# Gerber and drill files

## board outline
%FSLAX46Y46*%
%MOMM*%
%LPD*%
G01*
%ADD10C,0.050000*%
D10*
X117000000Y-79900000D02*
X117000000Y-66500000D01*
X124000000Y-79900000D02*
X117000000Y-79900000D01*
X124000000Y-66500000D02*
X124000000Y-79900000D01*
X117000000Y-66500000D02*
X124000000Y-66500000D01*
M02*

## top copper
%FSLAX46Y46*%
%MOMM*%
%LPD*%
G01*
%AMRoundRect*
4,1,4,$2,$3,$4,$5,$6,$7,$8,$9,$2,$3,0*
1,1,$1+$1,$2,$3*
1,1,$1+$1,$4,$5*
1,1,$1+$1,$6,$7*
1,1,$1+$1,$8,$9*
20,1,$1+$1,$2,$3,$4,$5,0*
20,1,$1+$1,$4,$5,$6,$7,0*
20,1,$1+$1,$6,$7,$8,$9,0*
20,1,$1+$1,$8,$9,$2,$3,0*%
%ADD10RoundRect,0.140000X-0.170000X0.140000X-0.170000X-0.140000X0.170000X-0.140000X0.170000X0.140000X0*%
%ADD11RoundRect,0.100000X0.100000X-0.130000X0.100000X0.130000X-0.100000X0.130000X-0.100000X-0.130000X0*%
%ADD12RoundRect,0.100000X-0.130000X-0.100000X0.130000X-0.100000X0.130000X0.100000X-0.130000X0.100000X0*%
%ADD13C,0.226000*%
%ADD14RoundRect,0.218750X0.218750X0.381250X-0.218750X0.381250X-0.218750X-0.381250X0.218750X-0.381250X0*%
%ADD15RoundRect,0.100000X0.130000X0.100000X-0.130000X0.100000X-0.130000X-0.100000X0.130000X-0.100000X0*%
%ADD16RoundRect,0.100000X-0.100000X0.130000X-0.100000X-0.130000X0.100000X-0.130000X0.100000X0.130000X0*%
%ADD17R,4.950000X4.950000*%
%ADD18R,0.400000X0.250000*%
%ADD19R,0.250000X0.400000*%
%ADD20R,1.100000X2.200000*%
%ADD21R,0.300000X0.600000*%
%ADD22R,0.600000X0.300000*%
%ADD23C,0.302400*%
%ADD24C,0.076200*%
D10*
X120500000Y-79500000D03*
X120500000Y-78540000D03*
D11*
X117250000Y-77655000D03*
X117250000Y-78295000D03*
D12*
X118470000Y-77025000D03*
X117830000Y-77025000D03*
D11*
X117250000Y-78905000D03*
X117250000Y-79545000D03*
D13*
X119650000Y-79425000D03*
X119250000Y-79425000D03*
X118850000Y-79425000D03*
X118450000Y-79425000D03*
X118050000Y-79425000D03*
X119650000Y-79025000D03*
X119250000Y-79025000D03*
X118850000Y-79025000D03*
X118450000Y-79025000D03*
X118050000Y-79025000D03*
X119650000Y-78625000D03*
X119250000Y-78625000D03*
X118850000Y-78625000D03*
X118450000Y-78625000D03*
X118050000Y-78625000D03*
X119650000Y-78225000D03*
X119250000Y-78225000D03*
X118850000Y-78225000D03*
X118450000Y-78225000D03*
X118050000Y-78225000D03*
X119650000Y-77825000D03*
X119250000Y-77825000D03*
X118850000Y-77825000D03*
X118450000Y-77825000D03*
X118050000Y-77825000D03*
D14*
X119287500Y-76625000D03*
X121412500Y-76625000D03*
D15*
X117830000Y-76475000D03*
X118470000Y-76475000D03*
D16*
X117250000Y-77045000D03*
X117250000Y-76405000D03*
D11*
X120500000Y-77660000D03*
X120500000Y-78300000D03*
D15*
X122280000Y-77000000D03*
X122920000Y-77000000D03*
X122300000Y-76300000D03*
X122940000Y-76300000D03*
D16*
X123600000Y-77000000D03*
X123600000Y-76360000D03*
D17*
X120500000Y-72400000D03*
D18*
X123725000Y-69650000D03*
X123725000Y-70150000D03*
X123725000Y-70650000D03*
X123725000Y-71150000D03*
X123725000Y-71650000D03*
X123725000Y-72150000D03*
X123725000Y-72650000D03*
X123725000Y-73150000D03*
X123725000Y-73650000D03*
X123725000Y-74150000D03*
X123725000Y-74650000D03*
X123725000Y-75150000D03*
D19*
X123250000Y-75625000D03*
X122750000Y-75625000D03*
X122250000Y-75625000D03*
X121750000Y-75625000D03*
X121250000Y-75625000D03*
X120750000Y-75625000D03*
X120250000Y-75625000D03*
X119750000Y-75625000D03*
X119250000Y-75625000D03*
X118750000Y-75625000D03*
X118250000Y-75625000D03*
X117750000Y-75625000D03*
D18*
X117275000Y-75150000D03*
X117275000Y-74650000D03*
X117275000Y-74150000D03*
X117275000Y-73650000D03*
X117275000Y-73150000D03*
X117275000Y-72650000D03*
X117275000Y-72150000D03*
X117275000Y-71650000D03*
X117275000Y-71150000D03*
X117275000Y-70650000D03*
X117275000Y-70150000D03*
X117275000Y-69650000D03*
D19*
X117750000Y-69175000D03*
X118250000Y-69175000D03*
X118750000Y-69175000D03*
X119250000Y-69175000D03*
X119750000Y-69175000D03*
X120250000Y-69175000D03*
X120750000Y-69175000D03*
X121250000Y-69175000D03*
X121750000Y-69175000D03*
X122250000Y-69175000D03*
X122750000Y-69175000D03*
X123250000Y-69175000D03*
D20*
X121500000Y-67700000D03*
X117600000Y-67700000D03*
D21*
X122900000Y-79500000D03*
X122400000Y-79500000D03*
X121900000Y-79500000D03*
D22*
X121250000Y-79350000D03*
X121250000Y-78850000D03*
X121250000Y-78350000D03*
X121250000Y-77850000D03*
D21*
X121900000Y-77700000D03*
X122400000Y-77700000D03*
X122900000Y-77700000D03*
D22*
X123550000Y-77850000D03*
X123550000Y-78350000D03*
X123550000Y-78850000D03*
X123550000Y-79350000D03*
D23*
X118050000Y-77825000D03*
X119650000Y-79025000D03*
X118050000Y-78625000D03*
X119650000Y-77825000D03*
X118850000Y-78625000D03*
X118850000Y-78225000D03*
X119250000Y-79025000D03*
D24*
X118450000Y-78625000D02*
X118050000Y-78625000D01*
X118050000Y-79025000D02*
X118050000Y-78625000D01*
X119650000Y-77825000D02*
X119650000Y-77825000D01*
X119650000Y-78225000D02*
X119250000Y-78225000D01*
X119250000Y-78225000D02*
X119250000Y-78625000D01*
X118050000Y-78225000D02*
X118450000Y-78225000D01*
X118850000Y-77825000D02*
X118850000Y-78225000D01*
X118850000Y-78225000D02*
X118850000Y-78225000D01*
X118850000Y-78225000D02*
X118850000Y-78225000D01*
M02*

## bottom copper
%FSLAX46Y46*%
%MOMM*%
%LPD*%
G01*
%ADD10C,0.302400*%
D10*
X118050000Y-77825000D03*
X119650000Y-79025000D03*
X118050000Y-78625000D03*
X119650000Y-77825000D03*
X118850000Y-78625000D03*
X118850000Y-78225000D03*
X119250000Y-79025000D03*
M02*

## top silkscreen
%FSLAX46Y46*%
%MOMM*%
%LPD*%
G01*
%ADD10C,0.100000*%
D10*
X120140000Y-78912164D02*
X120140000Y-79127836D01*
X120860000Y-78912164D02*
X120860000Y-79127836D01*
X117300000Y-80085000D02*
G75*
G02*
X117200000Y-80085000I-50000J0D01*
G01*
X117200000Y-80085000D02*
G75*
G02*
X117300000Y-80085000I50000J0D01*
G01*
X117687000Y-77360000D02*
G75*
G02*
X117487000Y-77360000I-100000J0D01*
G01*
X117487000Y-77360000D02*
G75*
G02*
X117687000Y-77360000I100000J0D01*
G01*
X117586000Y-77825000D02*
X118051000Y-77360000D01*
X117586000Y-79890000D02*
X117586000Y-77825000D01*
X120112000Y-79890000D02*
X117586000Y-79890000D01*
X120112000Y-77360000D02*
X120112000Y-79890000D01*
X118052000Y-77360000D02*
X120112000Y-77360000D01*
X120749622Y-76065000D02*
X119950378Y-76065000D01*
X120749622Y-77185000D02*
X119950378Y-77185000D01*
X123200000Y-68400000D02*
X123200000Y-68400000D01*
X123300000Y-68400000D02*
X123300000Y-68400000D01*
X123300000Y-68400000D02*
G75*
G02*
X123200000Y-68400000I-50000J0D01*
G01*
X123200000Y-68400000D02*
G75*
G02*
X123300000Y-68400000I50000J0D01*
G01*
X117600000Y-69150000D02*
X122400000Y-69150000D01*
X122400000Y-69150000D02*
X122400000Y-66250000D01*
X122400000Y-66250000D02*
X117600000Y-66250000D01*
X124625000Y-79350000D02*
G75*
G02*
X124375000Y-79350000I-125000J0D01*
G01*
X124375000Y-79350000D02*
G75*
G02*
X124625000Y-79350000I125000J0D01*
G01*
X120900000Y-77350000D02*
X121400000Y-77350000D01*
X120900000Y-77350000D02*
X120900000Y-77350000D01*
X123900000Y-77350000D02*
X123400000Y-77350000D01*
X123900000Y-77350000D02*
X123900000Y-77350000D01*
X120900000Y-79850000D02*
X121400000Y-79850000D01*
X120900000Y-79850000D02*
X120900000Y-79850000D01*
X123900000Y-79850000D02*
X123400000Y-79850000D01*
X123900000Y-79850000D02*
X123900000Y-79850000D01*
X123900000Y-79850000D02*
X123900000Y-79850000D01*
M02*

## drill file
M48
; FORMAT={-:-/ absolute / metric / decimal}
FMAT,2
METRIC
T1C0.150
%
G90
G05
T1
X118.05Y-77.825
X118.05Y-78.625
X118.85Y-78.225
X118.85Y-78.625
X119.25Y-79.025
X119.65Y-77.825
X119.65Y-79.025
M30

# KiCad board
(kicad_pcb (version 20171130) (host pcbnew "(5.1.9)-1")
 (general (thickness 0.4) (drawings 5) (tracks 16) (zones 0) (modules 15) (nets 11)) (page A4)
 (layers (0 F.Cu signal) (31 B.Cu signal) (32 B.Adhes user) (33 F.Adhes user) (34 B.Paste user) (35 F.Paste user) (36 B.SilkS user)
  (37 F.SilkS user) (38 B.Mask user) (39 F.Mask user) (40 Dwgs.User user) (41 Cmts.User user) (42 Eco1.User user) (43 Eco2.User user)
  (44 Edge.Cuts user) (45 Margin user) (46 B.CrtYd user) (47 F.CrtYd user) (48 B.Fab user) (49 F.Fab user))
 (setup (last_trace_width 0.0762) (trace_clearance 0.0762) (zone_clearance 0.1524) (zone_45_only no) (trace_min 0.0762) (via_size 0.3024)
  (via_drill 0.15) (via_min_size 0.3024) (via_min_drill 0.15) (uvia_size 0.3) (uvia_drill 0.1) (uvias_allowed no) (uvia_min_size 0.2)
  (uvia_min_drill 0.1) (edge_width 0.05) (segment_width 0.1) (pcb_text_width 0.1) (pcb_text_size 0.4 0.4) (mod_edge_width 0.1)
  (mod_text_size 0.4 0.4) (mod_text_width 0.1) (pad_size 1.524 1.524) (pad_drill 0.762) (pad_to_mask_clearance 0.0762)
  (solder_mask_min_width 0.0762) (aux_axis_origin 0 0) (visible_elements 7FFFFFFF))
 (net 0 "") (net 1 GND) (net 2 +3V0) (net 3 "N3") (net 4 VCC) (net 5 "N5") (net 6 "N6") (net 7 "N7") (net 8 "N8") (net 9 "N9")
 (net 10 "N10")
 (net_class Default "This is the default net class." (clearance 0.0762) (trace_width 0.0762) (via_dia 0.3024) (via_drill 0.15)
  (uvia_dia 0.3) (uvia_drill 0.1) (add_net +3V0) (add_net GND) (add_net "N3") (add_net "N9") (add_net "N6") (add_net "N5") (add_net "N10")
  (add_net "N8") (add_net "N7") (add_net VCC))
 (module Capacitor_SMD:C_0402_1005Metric (layer F.Cu) (at 120.5 79.02 270)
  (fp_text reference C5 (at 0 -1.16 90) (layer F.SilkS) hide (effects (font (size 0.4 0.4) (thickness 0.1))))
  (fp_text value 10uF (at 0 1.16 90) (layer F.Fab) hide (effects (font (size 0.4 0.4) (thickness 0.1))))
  (fp_line (start -0.107836 0.36) (end 0.107836 0.36) (layer F.SilkS) (width 0.1))
  (fp_line (start -0.107836 -0.36) (end 0.107836 -0.36) (layer F.SilkS) (width 0.1))
  (pad 2 smd roundrect (at 0.48 0 270) (size 0.56 0.62) (layers F.Cu F.Paste F.Mask) (roundrect_rratio 0.25) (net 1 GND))
  (pad 1 smd roundrect (at -0.48 0 270) (size 0.56 0.62) (layers F.Cu F.Paste F.Mask) (roundrect_rratio 0.25) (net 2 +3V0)))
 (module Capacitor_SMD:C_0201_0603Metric (layer F.Cu) (at 117.25 77.975 90)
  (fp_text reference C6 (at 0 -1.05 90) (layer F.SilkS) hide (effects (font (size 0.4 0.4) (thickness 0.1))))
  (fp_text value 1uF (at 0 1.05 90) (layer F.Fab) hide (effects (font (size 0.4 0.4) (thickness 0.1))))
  (pad 2 smd roundrect (at 0.32 0 90) (size 0.46 0.4) (layers F.Cu F.Mask) (roundrect_rratio 0.25) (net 1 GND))
  (pad 1 smd roundrect (at -0.32 0 90) (size 0.46 0.4) (layers F.Cu F.Mask) (roundrect_rratio 0.25) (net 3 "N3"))
  (pad "" smd roundrect (at 0.345 0 90) (size 0.318 0.36) (layers F.Paste) (roundrect_rratio 0.25))
  (pad "" smd roundrect (at -0.345 0 90) (size 0.318 0.36) (layers F.Paste) (roundrect_rratio 0.25)))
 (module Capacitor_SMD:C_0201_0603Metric (layer F.Cu) (at 118.15 77.025)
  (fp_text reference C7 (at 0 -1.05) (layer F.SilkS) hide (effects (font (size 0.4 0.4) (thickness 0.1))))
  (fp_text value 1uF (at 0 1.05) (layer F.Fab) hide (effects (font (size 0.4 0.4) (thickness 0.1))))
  (pad 2 smd roundrect (at 0.32 0) (size 0.46 0.4) (layers F.Cu F.Mask) (roundrect_rratio 0.25) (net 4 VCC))
  (pad 1 smd roundrect (at -0.32 0) (size 0.46 0.4) (layers F.Cu F.Mask) (roundrect_rratio 0.25) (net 1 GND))
  (pad "" smd roundrect (at 0.345 0) (size 0.318 0.36) (layers F.Paste) (roundrect_rratio 0.25))
  (pad "" smd roundrect (at -0.345 0) (size 0.318 0.36) (layers F.Paste) (roundrect_rratio 0.25)))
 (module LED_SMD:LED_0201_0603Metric (layer F.Cu) (at 117.25 79.225 90)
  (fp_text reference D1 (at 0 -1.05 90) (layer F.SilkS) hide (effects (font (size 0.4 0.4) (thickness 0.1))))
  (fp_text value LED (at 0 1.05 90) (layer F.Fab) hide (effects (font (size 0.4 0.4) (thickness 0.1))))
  (fp_circle (center -0.86 0) (end -0.81 0) (layer F.SilkS) (width 0.1))
  (pad 2 smd roundrect (at 0.32 0 90) (size 0.46 0.4) (layers F.Cu F.Mask) (roundrect_rratio 0.25) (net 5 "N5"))
  (pad 1 smd roundrect (at -0.32 0 90) (size 0.46 0.4) (layers F.Cu F.Mask) (roundrect_rratio 0.25) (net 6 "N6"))
  (pad "" smd roundrect (at 0.345 0 90) (size 0.318 0.36) (layers F.Paste) (roundrect_rratio 0.25))
  (pad "" smd roundrect (at -0.345 0 90) (size 0.318 0.36) (layers F.Paste) (roundrect_rratio 0.25)))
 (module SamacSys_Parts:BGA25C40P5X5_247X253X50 (layer F.Cu) (at 118.85 78.625)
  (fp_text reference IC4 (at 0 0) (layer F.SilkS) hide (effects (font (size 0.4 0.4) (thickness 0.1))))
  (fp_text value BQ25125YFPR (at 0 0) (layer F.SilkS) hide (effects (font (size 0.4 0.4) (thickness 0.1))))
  (fp_circle (center -1.263 -1.265) (end -1.263 -1.165) (layer F.SilkS) (width 0.1))
  (fp_line (start -1.264 -0.8) (end -0.799 -1.265) (layer F.SilkS) (width 0.1))
  (fp_line (start -1.264 1.265) (end -1.264 -0.8) (layer F.SilkS) (width 0.1))
  (fp_line (start 1.262 1.265) (end -1.264 1.265) (layer F.SilkS) (width 0.1))
  (fp_line (start 1.262 -1.265) (end 1.262 1.265) (layer F.SilkS) (width 0.1))
  (fp_line (start -0.798 -1.265) (end 1.262 -1.265) (layer F.SilkS) (width 0.1))
  (pad E5 smd circle (at 0.8 0.8 90) (size 0.226 0.226) (layers F.Cu F.Paste F.Mask))
  (pad E4 smd circle (at 0.4 0.8 90) (size 0.226 0.226) (layers F.Cu F.Paste F.Mask))
  (pad E3 smd circle (at 0 0.8 90) (size 0.226 0.226) (layers F.Cu F.Paste F.Mask))
  (pad E2 smd circle (at -0.4 0.8 90) (size 0.226 0.226) (layers F.Cu F.Paste F.Mask))
  (pad E1 smd circle (at -0.8 0.8 90) (size 0.226 0.226) (layers F.Cu F.Paste F.Mask))
  (pad D5 smd circle (at 0.8 0.4 90) (size 0.226 0.226) (layers F.Cu F.Paste F.Mask) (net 1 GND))
  (pad D4 smd circle (at 0.4 0.4 90) (size 0.226 0.226) (layers F.Cu F.Paste F.Mask) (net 6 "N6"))
  (pad D3 smd circle (at 0 0.4 90) (size 0.226 0.226) (layers F.Cu F.Paste F.Mask))
  (pad D2 smd circle (at -0.4 0.4 90) (size 0.226 0.226) (layers F.Cu F.Paste F.Mask))
  (pad D1 smd circle (at -0.8 0.4 90) (size 0.226 0.226) (layers F.Cu F.Paste F.Mask) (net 1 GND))
  (pad C5 smd circle (at 0.8 0 90) (size 0.226 0.226) (layers F.Cu F.Paste F.Mask))
  (pad C4 smd circle (at 0.4 0 90) (size 0.226 0.226) (layers F.Cu F.Paste F.Mask) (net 2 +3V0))
  (pad C3 smd circle (at 0 0 90) (size 0.226 0.226) (layers F.Cu F.Paste F.Mask) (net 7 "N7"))
  (pad C2 smd circle (at -0.4 0 90) (size 0.226 0.226) (layers F.Cu F.Paste F.Mask) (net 1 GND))
  (pad C1 smd circle (at -0.8 0 90) (size 0.226 0.226) (layers F.Cu F.Paste F.Mask) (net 1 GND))
  (pad B5 smd circle (at 0.8 -0.4 90) (size 0.226 0.226) (layers F.Cu F.Paste F.Mask) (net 2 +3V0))
  (pad B4 smd circle (at 0.4 -0.4 90) (size 0.226 0.226) (layers F.Cu F.Paste F.Mask) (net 2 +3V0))
  (pad B3 smd circle (at 0 -0.4 90) (size 0.226 0.226) (layers F.Cu F.Paste F.Mask) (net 5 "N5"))
  (pad B2 smd circle (at -0.4 -0.4 90) (size 0.226 0.226) (layers F.Cu F.Paste F.Mask) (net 3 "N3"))
  (pad B1 smd circle (at -0.8 -0.4 90) (size 0.226 0.226) (layers F.Cu F.Paste F.Mask) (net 3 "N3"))
  (pad A5 smd circle (at 0.8 -0.8 90) (size 0.226 0.226) (layers F.Cu F.Paste F.Mask) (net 1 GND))
  (pad A4 smd circle (at 0.4 -0.8 90) (size 0.226 0.226) (layers F.Cu F.Paste F.Mask) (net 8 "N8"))
  (pad A3 smd circle (at 0 -0.8 90) (size 0.226 0.226) (layers F.Cu F.Paste F.Mask) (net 5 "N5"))
  (pad A2 smd circle (at -0.4 -0.8 90) (size 0.226 0.226) (layers F.Cu F.Paste F.Mask) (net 4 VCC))
  (pad A1 smd circle (at -0.8 -0.8 90) (size 0.226 0.226) (layers F.Cu F.Paste F.Mask) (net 1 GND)))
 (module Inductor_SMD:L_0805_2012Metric (layer F.Cu) (at 120.35 76.625 180)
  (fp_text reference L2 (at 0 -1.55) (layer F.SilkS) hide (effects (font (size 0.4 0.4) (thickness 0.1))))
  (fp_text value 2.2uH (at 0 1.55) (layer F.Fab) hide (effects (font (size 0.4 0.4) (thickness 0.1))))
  (fp_line (start -0.399622 0.56) (end 0.399622 0.56) (layer F.SilkS) (width 0.1))
  (fp_line (start -0.399622 -0.56) (end 0.399622 -0.56) (layer F.SilkS) (width 0.1))
  (pad 2 smd roundrect (at 1.0625 0 180) (size 0.875 1.2) (layers F.Cu F.Paste F.Mask) (roundrect_rratio 0.25) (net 8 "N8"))
  (pad 1 smd roundrect (at -1.0625 0 180) (size 0.875 1.2) (layers F.Cu F.Paste F.Mask) (roundrect_rratio 0.25) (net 2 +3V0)))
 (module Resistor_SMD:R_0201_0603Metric (layer F.Cu) (at 118.15 76.475 180)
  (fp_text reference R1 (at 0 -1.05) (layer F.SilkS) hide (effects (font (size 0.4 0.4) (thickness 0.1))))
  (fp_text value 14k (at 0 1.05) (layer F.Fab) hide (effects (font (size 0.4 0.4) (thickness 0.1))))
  (pad 2 smd roundrect (at 0.32 0 180) (size 0.46 0.4) (layers F.Cu F.Mask) (roundrect_rratio 0.25) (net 7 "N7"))
  (pad 1 smd roundrect (at -0.32 0 180) (size 0.46 0.4) (layers F.Cu F.Mask) (roundrect_rratio 0.25) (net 4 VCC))
  (pad "" smd roundrect (at 0.345 0 180) (size 0.318 0.36) (layers F.Paste) (roundrect_rratio 0.25))
  (pad "" smd roundrect (at -0.345 0 180) (size 0.318 0.36) (layers F.Paste) (roundrect_rratio 0.25)))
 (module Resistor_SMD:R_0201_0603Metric (layer F.Cu) (at 117.25 76.725 270)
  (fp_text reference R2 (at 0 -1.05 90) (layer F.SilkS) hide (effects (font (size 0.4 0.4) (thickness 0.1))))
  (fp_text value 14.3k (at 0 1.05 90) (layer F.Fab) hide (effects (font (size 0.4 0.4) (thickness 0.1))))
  (pad 2 smd roundrect (at 0.32 0 270) (size 0.46 0.4) (layers F.Cu F.Mask) (roundrect_rratio 0.25) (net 1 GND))
  (pad 1 smd roundrect (at -0.32 0 270) (size 0.46 0.4) (layers F.Cu F.Mask) (roundrect_rratio 0.25) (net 7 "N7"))
  (pad "" smd roundrect (at 0.345 0 270) (size 0.318 0.36) (layers F.Paste) (roundrect_rratio 0.25))
  (pad "" smd roundrect (at -0.345 0 270) (size 0.318 0.36) (layers F.Paste) (roundrect_rratio 0.25)))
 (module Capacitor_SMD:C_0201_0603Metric (layer F.Cu) (at 120.5 77.98 90)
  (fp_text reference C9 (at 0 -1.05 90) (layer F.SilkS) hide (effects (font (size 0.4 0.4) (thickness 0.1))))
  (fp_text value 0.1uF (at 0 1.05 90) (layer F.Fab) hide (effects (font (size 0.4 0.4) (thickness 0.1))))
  (pad 2 smd roundrect (at 0.32 0 90) (size 0.46 0.4) (layers F.Cu F.Mask) (roundrect_rratio 0.25) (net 1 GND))
  (pad 1 smd roundrect (at -0.32 0 90) (size 0.46 0.4) (layers F.Cu F.Mask) (roundrect_rratio 0.25) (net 2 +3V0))
  (pad "" smd roundrect (at 0.345 0 90) (size 0.318 0.36) (layers F.Paste) (roundrect_rratio 0.25))
  (pad "" smd roundrect (at -0.345 0 90) (size 0.318 0.36) (layers F.Paste) (roundrect_rratio 0.25)))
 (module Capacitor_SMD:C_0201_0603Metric (layer F.Cu) (at 122.6 77 180)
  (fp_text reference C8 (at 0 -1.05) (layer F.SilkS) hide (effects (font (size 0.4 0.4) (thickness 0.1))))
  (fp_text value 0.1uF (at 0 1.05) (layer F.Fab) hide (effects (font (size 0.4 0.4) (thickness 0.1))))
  (pad 2 smd roundrect (at 0.32 0 180) (size 0.46 0.4) (layers F.Cu F.Mask) (roundrect_rratio 0.25) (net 1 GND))
  (pad 1 smd roundrect (at -0.32 0 180) (size 0.46 0.4) (layers F.Cu F.Mask) (roundrect_rratio 0.25) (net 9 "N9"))
  (pad "" smd roundrect (at 0.345 0 180) (size 0.318 0.36) (layers F.Paste) (roundrect_rratio 0.25))
  (pad "" smd roundrect (at -0.345 0 180) (size 0.318 0.36) (layers F.Paste) (roundrect_rratio 0.25)))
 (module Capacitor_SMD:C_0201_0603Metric (layer F.Cu) (at 122.62 76.3 180)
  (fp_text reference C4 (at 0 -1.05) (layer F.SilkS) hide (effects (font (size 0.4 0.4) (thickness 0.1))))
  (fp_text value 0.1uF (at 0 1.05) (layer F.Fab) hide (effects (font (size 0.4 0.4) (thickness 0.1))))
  (pad 2 smd roundrect (at 0.32 0 180) (size 0.46 0.4) (layers F.Cu F.Mask) (roundrect_rratio 0.25) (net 1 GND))
  (pad 1 smd roundrect (at -0.32 0 180) (size 0.46 0.4) (layers F.Cu F.Mask) (roundrect_rratio 0.25) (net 2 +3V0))
  (pad "" smd roundrect (at 0.345 0 180) (size 0.318 0.36) (layers F.Paste) (roundrect_rratio 0.25))
  (pad "" smd roundrect (at -0.345 0 180) (size 0.318 0.36) (layers F.Paste) (roundrect_rratio 0.25)))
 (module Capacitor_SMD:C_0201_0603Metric (layer F.Cu) (at 123.6 76.68 270)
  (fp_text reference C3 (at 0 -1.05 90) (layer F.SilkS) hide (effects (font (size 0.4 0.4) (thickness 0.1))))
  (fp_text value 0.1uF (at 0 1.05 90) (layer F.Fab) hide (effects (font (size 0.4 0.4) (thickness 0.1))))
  (pad 2 smd roundrect (at 0.32 0 270) (size 0.46 0.4) (layers F.Cu F.Mask) (roundrect_rratio 0.25) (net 1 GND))
  (pad 1 smd roundrect (at -0.32 0 270) (size 0.46 0.4) (layers F.Cu F.Mask) (roundrect_rratio 0.25) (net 2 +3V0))
  (pad "" smd roundrect (at 0.345 0 270) (size 0.318 0.36) (layers F.Paste) (roundrect_rratio 0.25))
  (pad "" smd roundrect (at -0.345 0 270) (size 0.318 0.36) (layers F.Paste) (roundrect_rratio 0.25)))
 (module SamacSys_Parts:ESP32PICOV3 (layer F.Cu) (at 120.5 72.4 270)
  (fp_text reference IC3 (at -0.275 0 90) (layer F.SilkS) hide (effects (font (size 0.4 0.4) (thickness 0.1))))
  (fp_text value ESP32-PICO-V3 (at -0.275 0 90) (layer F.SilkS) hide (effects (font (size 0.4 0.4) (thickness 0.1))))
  (fp_line (start -4 -2.7) (end -4 -2.7) (layer F.SilkS) (width 0.1))
  (fp_line (start -4 -2.8) (end -4 -2.8) (layer F.SilkS) (width 0.1))
  (fp_arc (start -4 -2.75) (end -4 -2.7) (angle -180) (layer F.SilkS) (width 0.1))
  (fp_arc (start -4 -2.75) (end -4 -2.8) (angle -180) (layer F.SilkS) (width 0.1))
  (pad 49 smd rect (at 0 0 270) (size 4.95 4.95) (layers F.Cu F.Paste F.Mask) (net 1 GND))
  (pad 48 smd rect (at -2.75 -3.225 270) (size 0.25 0.4) (layers F.Cu F.Paste F.Mask))
  (pad 47 smd rect (at -2.25 -3.225 270) (size 0.25 0.4) (layers F.Cu F.Paste F.Mask))
  (pad 46 smd rect (at -1.75 -3.225 270) (size 0.25 0.4) (layers F.Cu F.Paste F.Mask) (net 2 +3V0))
  (pad 45 smd rect (at -1.25 -3.225 270) (size 0.25 0.4) (layers F.Cu F.Paste F.Mask))
  (pad 44 smd rect (at -0.75 -3.225 270) (size 0.25 0.4) (layers F.Cu F.Paste F.Mask))
  (pad 43 smd rect (at -0.25 -3.225 270) (size 0.25 0.4) (layers F.Cu F.Paste F.Mask) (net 2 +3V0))
  (pad 42 smd rect (at 0.25 -3.225 270) (size 0.25 0.4) (layers F.Cu F.Paste F.Mask))
  (pad 41 smd rect (at 0.75 -3.225 270) (size 0.25 0.4) (layers F.Cu F.Paste F.Mask))
  (pad 40 smd rect (at 1.25 -3.225 270) (size 0.25 0.4) (layers F.Cu F.Paste F.Mask))
  (pad 39 smd rect (at 1.75 -3.225 270) (size 0.25 0.4) (layers F.Cu F.Paste F.Mask))
  (pad 38 smd rect (at 2.25 -3.225 270) (size 0.25 0.4) (layers F.Cu F.Paste F.Mask))
  (pad 37 smd rect (at 2.75 -3.225 270) (size 0.25 0.4) (layers F.Cu F.Paste F.Mask) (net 2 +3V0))
  (pad 36 smd rect (at 3.225 -2.75) (size 0.25 0.4) (layers F.Cu F.Paste F.Mask))
  (pad 35 smd rect (at 3.225 -2.25) (size 0.25 0.4) (layers F.Cu F.Paste F.Mask))
  (pad 34 smd rect (at 3.225 -1.75) (size 0.25 0.4) (layers F.Cu F.Paste F.Mask))
  (pad 33 smd rect (at 3.225 -1.25) (size 0.25 0.4) (layers F.Cu F.Paste F.Mask))
  (pad 32 smd rect (at 3.225 -0.75) (size 0.25 0.4) (layers F.Cu F.Paste F.Mask))
  (pad 31 smd rect (at 3.225 -0.25) (size 0.25 0.4) (layers F.Cu F.Paste F.Mask))
  (pad 30 smd rect (at 3.225 0.25) (size 0.25 0.4) (layers F.Cu F.Paste F.Mask))
  (pad 29 smd rect (at 3.225 0.75) (size 0.25 0.4) (layers F.Cu F.Paste F.Mask))
  (pad 28 smd rect (at 3.225 1.25) (size 0.25 0.4) (layers F.Cu F.Paste F.Mask))
  (pad 27 smd rect (at 3.225 1.75) (size 0.25 0.4) (layers F.Cu F.Paste F.Mask))
  (pad 26 smd rect (at 3.225 2.25) (size 0.25 0.4) (layers F.Cu F.Paste F.Mask))
  (pad 25 smd rect (at 3.225 2.75) (size 0.25 0.4) (layers F.Cu F.Paste F.Mask))
  (pad 24 smd rect (at 2.75 3.225 270) (size 0.25 0.4) (layers F.Cu F.Paste F.Mask))
  (pad 23 smd rect (at 2.25 3.225 270) (size 0.25 0.4) (layers F.Cu F.Paste F.Mask))
  (pad 22 smd rect (at 1.75 3.225 270) (size 0.25 0.4) (layers F.Cu F.Paste F.Mask))
  (pad 21 smd rect (at 1.25 3.225 270) (size 0.25 0.4) (layers F.Cu F.Paste F.Mask))
  (pad 20 smd rect (at 0.75 3.225 270) (size 0.25 0.4) (layers F.Cu F.Paste F.Mask))
  (pad 19 smd rect (at 0.25 3.225 270) (size 0.25 0.4) (layers F.Cu F.Paste F.Mask) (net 2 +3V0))
  (pad 18 smd rect (at -0.25 3.225 270) (size 0.25 0.4) (layers F.Cu F.Paste F.Mask))
  (pad 17 smd rect (at -0.75 3.225 270) (size 0.25 0.4) (layers F.Cu F.Paste F.Mask))
  (pad 16 smd rect (at -1.25 3.225 270) (size 0.25 0.4) (layers F.Cu F.Paste F.Mask))
  (pad 15 smd rect (at -1.75 3.225 270) (size 0.25 0.4) (layers F.Cu F.Paste F.Mask))
  (pad 14 smd rect (at -2.25 3.225 270) (size 0.25 0.4) (layers F.Cu F.Paste F.Mask))
  (pad 13 smd rect (at -2.75 3.225 270) (size 0.25 0.4) (layers F.Cu F.Paste F.Mask))
  (pad 12 smd rect (at -3.225 2.75) (size 0.25 0.4) (layers F.Cu F.Paste F.Mask))
  (pad 11 smd rect (at -3.225 2.25) (size 0.25 0.4) (layers F.Cu F.Paste F.Mask))
  (pad 10 smd rect (at -3.225 1.75) (size 0.25 0.4) (layers F.Cu F.Paste F.Mask))
  (pad 9 smd rect (at -3.225 1.25) (size 0.25 0.4) (layers F.Cu F.Paste F.Mask))
  (pad 8 smd rect (at -3.225 0.75) (size 0.25 0.4) (layers F.Cu F.Paste F.Mask))
  (pad 7 smd rect (at -3.225 0.25) (size 0.25 0.4) (layers F.Cu F.Paste F.Mask))
  (pad 6 smd rect (at -3.225 -0.25) (size 0.25 0.4) (layers F.Cu F.Paste F.Mask))
  (pad 5 smd rect (at -3.225 -0.75) (size 0.25 0.4) (layers F.Cu F.Paste F.Mask))
  (pad 4 smd rect (at -3.225 -1.25) (size 0.25 0.4) (layers F.Cu F.Paste F.Mask) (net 2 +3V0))
  (pad 3 smd rect (at -3.225 -1.75) (size 0.25 0.4) (layers F.Cu F.Paste F.Mask) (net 2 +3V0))
  (pad 2 smd rect (at -3.225 -2.25) (size 0.25 0.4) (layers F.Cu F.Paste F.Mask) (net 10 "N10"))
  (pad 1 smd rect (at -3.225 -2.75) (size 0.25 0.4) (layers F.Cu F.Paste F.Mask) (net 2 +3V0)))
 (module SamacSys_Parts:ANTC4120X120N (layer F.Cu) (at 119.55 67.7 180)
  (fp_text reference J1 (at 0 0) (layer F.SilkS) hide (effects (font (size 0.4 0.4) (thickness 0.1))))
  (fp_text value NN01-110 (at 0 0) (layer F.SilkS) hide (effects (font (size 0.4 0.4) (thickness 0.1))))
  (fp_line (start 1.95 -1.45) (end -2.85 -1.45) (layer F.SilkS) (width 0.1))
  (fp_line (start -2.85 -1.45) (end -2.85 1.45) (layer F.SilkS) (width 0.1))
  (fp_line (start -2.85 1.45) (end 1.95 1.45) (layer F.SilkS) (width 0.1))
  (pad 1 smd rect (at -1.95 0 180) (size 1.1 2.2) (layers F.Cu F.Paste F.Mask) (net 10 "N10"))
  (pad 2 smd rect (at 1.95 0 180) (size 1.1 2.2) (layers F.Cu F.Paste F.Mask)))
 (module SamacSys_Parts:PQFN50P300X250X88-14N (layer F.Cu) (at 122.4 78.6 180)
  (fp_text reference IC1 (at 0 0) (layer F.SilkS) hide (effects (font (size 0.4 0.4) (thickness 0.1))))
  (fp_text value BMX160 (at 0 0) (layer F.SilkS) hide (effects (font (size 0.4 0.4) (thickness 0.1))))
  (fp_circle (center -2.1 -0.75) (end -2.1 -0.625) (layer F.SilkS) (width 0.1))
  (fp_line (start 1.5 1.25) (end 1 1.25) (layer F.SilkS) (width 0.1))
  (fp_line (start 1.5 1.25) (end 1.5 1.25) (layer F.SilkS) (width 0.1))
  (fp_line (start -1.5 1.25) (end -1 1.25) (layer F.SilkS) (width 0.1))
  (fp_line (start -1.5 1.25) (end -1.5 1.25) (layer F.SilkS) (width 0.1))
  (fp_line (start 1.5 -1.25) (end 1 -1.25) (layer F.SilkS) (width 0.1))
  (fp_line (start 1.5 -1.25) (end 1.5 -1.25) (layer F.SilkS) (width 0.1))
  (fp_line (start -1.5 -1.25) (end -1 -1.25) (layer F.SilkS) (width 0.1))
  (fp_line (start -1.5 -1.25) (end -1.5 -1.25) (layer F.SilkS) (width 0.1))
  (fp_line (start -1.5 -1.25) (end -1.5 -1.25) (layer F.SilkS) (width 0.1))
  (pad 14 smd rect (at -0.5 -0.9 180) (size 0.3 0.6) (layers F.Cu F.Paste F.Mask))
  (pad 13 smd rect (at 0 -0.9 180) (size 0.3 0.6) (layers F.Cu F.Paste F.Mask))
  (pad 12 smd rect (at 0.5 -0.9 180) (size 0.3 0.6) (layers F.Cu F.Paste F.Mask))
  (pad 11 smd rect (at 1.15 -0.75 270) (size 0.3 0.6) (layers F.Cu F.Paste F.Mask))
  (pad 10 smd rect (at 1.15 -0.25 270) (size 0.3 0.6) (layers F.Cu F.Paste F.Mask))
  (pad 9 smd rect (at 1.15 0.25 270) (size 0.3 0.6) (layers F.Cu F.Paste F.Mask))
  (pad 8 smd rect (at 1.15 0.75 270) (size 0.3 0.6) (layers F.Cu F.Paste F.Mask) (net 2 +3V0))
  (pad 7 smd rect (at 0.5 0.9 180) (size 0.3 0.6) (layers F.Cu F.Paste F.Mask) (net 1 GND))
  (pad 6 smd rect (at 0 0.9 180) (size 0.3 0.6) (layers F.Cu F.Paste F.Mask) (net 1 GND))
  (pad 5 smd rect (at -0.5 0.9 180) (size 0.3 0.6) (layers F.Cu F.Paste F.Mask) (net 9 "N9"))
  (pad 4 smd rect (at -1.15 0.75 270) (size 0.3 0.6) (layers F.Cu F.Paste F.Mask))
  (pad 3 smd rect (at -1.15 0.25 270) (size 0.3 0.6) (layers F.Cu F.Paste F.Mask) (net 1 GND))
  (pad 2 smd rect (at -1.15 -0.25 270) (size 0.3 0.6) (layers F.Cu F.Paste F.Mask) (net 1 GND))
  (pad 1 smd rect (at -1.15 -0.75 270) (size 0.3 0.6) (layers F.Cu F.Paste F.Mask)))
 (gr_line (start 117 79.9) (end 117 66.5) (layer Edge.Cuts) (width 0.05))
 (gr_line (start 124 79.9) (end 117 79.9) (layer Edge.Cuts) (width 0.05))
 (gr_line (start 124 66.5) (end 124 79.9) (layer Edge.Cuts) (width 0.05))
 (gr_line (start 117 66.5) (end 124 66.5) (layer Edge.Cuts) (width 0.05))
 (via (at 118.05 77.825) (size 0.3024) (drill 0.15) (layers F.Cu B.Cu) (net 1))
 (via (at 119.65 79.025) (size 0.3024) (drill 0.15) (layers F.Cu B.Cu) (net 1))
 (segment (start 118.45 78.625) (end 118.05 78.625) (width 0.0762) (layer F.Cu) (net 1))
 (segment (start 118.05 79.025) (end 118.05 78.625) (width 0.0762) (layer F.Cu) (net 1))
 (via (at 118.05 78.625) (size 0.3024) (drill 0.15) (layers F.Cu B.Cu) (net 1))
 (via (at 119.65 77.825) (size 0.3024) (drill 0.15) (layers F.Cu B.Cu) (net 1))
 (segment (start 119.65 77.825) (end 119.65 77.825) (width 0.0762) (layer F.Cu) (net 1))
 (segment (start 119.65 78.225) (end 119.25 78.225) (width 0.0762) (layer F.Cu) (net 2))
 (segment (start 119.25 78.225) (end 119.25 78.625) (width 0.0762) (layer F.Cu) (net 2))
 (via (at 118.85 78.625) (size 0.3024) (drill 0.15) (layers F.Cu B.Cu) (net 7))
 (segment (start 118.05 78.225) (end 118.45 78.225) (width 0.0762) (layer F.Cu) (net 3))
 (segment (start 118.85 77.825) (end 118.85 78.225) (width 0.0762) (layer F.Cu) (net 5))
 (segment (start 118.85 78.225) (end 118.85 78.225) (width 0.0762) (layer F.Cu) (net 5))
 (segment (start 118.85 78.225) (end 118.85 78.225) (width 0.0762) (layer F.Cu) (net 5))
 (via (at 118.85 78.225) (size 0.3024) (drill 0.15) (layers F.Cu B.Cu) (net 5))
 (via (at 119.25 79.025) (size 0.3024) (drill 0.15) (layers F.Cu B.Cu) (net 6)))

